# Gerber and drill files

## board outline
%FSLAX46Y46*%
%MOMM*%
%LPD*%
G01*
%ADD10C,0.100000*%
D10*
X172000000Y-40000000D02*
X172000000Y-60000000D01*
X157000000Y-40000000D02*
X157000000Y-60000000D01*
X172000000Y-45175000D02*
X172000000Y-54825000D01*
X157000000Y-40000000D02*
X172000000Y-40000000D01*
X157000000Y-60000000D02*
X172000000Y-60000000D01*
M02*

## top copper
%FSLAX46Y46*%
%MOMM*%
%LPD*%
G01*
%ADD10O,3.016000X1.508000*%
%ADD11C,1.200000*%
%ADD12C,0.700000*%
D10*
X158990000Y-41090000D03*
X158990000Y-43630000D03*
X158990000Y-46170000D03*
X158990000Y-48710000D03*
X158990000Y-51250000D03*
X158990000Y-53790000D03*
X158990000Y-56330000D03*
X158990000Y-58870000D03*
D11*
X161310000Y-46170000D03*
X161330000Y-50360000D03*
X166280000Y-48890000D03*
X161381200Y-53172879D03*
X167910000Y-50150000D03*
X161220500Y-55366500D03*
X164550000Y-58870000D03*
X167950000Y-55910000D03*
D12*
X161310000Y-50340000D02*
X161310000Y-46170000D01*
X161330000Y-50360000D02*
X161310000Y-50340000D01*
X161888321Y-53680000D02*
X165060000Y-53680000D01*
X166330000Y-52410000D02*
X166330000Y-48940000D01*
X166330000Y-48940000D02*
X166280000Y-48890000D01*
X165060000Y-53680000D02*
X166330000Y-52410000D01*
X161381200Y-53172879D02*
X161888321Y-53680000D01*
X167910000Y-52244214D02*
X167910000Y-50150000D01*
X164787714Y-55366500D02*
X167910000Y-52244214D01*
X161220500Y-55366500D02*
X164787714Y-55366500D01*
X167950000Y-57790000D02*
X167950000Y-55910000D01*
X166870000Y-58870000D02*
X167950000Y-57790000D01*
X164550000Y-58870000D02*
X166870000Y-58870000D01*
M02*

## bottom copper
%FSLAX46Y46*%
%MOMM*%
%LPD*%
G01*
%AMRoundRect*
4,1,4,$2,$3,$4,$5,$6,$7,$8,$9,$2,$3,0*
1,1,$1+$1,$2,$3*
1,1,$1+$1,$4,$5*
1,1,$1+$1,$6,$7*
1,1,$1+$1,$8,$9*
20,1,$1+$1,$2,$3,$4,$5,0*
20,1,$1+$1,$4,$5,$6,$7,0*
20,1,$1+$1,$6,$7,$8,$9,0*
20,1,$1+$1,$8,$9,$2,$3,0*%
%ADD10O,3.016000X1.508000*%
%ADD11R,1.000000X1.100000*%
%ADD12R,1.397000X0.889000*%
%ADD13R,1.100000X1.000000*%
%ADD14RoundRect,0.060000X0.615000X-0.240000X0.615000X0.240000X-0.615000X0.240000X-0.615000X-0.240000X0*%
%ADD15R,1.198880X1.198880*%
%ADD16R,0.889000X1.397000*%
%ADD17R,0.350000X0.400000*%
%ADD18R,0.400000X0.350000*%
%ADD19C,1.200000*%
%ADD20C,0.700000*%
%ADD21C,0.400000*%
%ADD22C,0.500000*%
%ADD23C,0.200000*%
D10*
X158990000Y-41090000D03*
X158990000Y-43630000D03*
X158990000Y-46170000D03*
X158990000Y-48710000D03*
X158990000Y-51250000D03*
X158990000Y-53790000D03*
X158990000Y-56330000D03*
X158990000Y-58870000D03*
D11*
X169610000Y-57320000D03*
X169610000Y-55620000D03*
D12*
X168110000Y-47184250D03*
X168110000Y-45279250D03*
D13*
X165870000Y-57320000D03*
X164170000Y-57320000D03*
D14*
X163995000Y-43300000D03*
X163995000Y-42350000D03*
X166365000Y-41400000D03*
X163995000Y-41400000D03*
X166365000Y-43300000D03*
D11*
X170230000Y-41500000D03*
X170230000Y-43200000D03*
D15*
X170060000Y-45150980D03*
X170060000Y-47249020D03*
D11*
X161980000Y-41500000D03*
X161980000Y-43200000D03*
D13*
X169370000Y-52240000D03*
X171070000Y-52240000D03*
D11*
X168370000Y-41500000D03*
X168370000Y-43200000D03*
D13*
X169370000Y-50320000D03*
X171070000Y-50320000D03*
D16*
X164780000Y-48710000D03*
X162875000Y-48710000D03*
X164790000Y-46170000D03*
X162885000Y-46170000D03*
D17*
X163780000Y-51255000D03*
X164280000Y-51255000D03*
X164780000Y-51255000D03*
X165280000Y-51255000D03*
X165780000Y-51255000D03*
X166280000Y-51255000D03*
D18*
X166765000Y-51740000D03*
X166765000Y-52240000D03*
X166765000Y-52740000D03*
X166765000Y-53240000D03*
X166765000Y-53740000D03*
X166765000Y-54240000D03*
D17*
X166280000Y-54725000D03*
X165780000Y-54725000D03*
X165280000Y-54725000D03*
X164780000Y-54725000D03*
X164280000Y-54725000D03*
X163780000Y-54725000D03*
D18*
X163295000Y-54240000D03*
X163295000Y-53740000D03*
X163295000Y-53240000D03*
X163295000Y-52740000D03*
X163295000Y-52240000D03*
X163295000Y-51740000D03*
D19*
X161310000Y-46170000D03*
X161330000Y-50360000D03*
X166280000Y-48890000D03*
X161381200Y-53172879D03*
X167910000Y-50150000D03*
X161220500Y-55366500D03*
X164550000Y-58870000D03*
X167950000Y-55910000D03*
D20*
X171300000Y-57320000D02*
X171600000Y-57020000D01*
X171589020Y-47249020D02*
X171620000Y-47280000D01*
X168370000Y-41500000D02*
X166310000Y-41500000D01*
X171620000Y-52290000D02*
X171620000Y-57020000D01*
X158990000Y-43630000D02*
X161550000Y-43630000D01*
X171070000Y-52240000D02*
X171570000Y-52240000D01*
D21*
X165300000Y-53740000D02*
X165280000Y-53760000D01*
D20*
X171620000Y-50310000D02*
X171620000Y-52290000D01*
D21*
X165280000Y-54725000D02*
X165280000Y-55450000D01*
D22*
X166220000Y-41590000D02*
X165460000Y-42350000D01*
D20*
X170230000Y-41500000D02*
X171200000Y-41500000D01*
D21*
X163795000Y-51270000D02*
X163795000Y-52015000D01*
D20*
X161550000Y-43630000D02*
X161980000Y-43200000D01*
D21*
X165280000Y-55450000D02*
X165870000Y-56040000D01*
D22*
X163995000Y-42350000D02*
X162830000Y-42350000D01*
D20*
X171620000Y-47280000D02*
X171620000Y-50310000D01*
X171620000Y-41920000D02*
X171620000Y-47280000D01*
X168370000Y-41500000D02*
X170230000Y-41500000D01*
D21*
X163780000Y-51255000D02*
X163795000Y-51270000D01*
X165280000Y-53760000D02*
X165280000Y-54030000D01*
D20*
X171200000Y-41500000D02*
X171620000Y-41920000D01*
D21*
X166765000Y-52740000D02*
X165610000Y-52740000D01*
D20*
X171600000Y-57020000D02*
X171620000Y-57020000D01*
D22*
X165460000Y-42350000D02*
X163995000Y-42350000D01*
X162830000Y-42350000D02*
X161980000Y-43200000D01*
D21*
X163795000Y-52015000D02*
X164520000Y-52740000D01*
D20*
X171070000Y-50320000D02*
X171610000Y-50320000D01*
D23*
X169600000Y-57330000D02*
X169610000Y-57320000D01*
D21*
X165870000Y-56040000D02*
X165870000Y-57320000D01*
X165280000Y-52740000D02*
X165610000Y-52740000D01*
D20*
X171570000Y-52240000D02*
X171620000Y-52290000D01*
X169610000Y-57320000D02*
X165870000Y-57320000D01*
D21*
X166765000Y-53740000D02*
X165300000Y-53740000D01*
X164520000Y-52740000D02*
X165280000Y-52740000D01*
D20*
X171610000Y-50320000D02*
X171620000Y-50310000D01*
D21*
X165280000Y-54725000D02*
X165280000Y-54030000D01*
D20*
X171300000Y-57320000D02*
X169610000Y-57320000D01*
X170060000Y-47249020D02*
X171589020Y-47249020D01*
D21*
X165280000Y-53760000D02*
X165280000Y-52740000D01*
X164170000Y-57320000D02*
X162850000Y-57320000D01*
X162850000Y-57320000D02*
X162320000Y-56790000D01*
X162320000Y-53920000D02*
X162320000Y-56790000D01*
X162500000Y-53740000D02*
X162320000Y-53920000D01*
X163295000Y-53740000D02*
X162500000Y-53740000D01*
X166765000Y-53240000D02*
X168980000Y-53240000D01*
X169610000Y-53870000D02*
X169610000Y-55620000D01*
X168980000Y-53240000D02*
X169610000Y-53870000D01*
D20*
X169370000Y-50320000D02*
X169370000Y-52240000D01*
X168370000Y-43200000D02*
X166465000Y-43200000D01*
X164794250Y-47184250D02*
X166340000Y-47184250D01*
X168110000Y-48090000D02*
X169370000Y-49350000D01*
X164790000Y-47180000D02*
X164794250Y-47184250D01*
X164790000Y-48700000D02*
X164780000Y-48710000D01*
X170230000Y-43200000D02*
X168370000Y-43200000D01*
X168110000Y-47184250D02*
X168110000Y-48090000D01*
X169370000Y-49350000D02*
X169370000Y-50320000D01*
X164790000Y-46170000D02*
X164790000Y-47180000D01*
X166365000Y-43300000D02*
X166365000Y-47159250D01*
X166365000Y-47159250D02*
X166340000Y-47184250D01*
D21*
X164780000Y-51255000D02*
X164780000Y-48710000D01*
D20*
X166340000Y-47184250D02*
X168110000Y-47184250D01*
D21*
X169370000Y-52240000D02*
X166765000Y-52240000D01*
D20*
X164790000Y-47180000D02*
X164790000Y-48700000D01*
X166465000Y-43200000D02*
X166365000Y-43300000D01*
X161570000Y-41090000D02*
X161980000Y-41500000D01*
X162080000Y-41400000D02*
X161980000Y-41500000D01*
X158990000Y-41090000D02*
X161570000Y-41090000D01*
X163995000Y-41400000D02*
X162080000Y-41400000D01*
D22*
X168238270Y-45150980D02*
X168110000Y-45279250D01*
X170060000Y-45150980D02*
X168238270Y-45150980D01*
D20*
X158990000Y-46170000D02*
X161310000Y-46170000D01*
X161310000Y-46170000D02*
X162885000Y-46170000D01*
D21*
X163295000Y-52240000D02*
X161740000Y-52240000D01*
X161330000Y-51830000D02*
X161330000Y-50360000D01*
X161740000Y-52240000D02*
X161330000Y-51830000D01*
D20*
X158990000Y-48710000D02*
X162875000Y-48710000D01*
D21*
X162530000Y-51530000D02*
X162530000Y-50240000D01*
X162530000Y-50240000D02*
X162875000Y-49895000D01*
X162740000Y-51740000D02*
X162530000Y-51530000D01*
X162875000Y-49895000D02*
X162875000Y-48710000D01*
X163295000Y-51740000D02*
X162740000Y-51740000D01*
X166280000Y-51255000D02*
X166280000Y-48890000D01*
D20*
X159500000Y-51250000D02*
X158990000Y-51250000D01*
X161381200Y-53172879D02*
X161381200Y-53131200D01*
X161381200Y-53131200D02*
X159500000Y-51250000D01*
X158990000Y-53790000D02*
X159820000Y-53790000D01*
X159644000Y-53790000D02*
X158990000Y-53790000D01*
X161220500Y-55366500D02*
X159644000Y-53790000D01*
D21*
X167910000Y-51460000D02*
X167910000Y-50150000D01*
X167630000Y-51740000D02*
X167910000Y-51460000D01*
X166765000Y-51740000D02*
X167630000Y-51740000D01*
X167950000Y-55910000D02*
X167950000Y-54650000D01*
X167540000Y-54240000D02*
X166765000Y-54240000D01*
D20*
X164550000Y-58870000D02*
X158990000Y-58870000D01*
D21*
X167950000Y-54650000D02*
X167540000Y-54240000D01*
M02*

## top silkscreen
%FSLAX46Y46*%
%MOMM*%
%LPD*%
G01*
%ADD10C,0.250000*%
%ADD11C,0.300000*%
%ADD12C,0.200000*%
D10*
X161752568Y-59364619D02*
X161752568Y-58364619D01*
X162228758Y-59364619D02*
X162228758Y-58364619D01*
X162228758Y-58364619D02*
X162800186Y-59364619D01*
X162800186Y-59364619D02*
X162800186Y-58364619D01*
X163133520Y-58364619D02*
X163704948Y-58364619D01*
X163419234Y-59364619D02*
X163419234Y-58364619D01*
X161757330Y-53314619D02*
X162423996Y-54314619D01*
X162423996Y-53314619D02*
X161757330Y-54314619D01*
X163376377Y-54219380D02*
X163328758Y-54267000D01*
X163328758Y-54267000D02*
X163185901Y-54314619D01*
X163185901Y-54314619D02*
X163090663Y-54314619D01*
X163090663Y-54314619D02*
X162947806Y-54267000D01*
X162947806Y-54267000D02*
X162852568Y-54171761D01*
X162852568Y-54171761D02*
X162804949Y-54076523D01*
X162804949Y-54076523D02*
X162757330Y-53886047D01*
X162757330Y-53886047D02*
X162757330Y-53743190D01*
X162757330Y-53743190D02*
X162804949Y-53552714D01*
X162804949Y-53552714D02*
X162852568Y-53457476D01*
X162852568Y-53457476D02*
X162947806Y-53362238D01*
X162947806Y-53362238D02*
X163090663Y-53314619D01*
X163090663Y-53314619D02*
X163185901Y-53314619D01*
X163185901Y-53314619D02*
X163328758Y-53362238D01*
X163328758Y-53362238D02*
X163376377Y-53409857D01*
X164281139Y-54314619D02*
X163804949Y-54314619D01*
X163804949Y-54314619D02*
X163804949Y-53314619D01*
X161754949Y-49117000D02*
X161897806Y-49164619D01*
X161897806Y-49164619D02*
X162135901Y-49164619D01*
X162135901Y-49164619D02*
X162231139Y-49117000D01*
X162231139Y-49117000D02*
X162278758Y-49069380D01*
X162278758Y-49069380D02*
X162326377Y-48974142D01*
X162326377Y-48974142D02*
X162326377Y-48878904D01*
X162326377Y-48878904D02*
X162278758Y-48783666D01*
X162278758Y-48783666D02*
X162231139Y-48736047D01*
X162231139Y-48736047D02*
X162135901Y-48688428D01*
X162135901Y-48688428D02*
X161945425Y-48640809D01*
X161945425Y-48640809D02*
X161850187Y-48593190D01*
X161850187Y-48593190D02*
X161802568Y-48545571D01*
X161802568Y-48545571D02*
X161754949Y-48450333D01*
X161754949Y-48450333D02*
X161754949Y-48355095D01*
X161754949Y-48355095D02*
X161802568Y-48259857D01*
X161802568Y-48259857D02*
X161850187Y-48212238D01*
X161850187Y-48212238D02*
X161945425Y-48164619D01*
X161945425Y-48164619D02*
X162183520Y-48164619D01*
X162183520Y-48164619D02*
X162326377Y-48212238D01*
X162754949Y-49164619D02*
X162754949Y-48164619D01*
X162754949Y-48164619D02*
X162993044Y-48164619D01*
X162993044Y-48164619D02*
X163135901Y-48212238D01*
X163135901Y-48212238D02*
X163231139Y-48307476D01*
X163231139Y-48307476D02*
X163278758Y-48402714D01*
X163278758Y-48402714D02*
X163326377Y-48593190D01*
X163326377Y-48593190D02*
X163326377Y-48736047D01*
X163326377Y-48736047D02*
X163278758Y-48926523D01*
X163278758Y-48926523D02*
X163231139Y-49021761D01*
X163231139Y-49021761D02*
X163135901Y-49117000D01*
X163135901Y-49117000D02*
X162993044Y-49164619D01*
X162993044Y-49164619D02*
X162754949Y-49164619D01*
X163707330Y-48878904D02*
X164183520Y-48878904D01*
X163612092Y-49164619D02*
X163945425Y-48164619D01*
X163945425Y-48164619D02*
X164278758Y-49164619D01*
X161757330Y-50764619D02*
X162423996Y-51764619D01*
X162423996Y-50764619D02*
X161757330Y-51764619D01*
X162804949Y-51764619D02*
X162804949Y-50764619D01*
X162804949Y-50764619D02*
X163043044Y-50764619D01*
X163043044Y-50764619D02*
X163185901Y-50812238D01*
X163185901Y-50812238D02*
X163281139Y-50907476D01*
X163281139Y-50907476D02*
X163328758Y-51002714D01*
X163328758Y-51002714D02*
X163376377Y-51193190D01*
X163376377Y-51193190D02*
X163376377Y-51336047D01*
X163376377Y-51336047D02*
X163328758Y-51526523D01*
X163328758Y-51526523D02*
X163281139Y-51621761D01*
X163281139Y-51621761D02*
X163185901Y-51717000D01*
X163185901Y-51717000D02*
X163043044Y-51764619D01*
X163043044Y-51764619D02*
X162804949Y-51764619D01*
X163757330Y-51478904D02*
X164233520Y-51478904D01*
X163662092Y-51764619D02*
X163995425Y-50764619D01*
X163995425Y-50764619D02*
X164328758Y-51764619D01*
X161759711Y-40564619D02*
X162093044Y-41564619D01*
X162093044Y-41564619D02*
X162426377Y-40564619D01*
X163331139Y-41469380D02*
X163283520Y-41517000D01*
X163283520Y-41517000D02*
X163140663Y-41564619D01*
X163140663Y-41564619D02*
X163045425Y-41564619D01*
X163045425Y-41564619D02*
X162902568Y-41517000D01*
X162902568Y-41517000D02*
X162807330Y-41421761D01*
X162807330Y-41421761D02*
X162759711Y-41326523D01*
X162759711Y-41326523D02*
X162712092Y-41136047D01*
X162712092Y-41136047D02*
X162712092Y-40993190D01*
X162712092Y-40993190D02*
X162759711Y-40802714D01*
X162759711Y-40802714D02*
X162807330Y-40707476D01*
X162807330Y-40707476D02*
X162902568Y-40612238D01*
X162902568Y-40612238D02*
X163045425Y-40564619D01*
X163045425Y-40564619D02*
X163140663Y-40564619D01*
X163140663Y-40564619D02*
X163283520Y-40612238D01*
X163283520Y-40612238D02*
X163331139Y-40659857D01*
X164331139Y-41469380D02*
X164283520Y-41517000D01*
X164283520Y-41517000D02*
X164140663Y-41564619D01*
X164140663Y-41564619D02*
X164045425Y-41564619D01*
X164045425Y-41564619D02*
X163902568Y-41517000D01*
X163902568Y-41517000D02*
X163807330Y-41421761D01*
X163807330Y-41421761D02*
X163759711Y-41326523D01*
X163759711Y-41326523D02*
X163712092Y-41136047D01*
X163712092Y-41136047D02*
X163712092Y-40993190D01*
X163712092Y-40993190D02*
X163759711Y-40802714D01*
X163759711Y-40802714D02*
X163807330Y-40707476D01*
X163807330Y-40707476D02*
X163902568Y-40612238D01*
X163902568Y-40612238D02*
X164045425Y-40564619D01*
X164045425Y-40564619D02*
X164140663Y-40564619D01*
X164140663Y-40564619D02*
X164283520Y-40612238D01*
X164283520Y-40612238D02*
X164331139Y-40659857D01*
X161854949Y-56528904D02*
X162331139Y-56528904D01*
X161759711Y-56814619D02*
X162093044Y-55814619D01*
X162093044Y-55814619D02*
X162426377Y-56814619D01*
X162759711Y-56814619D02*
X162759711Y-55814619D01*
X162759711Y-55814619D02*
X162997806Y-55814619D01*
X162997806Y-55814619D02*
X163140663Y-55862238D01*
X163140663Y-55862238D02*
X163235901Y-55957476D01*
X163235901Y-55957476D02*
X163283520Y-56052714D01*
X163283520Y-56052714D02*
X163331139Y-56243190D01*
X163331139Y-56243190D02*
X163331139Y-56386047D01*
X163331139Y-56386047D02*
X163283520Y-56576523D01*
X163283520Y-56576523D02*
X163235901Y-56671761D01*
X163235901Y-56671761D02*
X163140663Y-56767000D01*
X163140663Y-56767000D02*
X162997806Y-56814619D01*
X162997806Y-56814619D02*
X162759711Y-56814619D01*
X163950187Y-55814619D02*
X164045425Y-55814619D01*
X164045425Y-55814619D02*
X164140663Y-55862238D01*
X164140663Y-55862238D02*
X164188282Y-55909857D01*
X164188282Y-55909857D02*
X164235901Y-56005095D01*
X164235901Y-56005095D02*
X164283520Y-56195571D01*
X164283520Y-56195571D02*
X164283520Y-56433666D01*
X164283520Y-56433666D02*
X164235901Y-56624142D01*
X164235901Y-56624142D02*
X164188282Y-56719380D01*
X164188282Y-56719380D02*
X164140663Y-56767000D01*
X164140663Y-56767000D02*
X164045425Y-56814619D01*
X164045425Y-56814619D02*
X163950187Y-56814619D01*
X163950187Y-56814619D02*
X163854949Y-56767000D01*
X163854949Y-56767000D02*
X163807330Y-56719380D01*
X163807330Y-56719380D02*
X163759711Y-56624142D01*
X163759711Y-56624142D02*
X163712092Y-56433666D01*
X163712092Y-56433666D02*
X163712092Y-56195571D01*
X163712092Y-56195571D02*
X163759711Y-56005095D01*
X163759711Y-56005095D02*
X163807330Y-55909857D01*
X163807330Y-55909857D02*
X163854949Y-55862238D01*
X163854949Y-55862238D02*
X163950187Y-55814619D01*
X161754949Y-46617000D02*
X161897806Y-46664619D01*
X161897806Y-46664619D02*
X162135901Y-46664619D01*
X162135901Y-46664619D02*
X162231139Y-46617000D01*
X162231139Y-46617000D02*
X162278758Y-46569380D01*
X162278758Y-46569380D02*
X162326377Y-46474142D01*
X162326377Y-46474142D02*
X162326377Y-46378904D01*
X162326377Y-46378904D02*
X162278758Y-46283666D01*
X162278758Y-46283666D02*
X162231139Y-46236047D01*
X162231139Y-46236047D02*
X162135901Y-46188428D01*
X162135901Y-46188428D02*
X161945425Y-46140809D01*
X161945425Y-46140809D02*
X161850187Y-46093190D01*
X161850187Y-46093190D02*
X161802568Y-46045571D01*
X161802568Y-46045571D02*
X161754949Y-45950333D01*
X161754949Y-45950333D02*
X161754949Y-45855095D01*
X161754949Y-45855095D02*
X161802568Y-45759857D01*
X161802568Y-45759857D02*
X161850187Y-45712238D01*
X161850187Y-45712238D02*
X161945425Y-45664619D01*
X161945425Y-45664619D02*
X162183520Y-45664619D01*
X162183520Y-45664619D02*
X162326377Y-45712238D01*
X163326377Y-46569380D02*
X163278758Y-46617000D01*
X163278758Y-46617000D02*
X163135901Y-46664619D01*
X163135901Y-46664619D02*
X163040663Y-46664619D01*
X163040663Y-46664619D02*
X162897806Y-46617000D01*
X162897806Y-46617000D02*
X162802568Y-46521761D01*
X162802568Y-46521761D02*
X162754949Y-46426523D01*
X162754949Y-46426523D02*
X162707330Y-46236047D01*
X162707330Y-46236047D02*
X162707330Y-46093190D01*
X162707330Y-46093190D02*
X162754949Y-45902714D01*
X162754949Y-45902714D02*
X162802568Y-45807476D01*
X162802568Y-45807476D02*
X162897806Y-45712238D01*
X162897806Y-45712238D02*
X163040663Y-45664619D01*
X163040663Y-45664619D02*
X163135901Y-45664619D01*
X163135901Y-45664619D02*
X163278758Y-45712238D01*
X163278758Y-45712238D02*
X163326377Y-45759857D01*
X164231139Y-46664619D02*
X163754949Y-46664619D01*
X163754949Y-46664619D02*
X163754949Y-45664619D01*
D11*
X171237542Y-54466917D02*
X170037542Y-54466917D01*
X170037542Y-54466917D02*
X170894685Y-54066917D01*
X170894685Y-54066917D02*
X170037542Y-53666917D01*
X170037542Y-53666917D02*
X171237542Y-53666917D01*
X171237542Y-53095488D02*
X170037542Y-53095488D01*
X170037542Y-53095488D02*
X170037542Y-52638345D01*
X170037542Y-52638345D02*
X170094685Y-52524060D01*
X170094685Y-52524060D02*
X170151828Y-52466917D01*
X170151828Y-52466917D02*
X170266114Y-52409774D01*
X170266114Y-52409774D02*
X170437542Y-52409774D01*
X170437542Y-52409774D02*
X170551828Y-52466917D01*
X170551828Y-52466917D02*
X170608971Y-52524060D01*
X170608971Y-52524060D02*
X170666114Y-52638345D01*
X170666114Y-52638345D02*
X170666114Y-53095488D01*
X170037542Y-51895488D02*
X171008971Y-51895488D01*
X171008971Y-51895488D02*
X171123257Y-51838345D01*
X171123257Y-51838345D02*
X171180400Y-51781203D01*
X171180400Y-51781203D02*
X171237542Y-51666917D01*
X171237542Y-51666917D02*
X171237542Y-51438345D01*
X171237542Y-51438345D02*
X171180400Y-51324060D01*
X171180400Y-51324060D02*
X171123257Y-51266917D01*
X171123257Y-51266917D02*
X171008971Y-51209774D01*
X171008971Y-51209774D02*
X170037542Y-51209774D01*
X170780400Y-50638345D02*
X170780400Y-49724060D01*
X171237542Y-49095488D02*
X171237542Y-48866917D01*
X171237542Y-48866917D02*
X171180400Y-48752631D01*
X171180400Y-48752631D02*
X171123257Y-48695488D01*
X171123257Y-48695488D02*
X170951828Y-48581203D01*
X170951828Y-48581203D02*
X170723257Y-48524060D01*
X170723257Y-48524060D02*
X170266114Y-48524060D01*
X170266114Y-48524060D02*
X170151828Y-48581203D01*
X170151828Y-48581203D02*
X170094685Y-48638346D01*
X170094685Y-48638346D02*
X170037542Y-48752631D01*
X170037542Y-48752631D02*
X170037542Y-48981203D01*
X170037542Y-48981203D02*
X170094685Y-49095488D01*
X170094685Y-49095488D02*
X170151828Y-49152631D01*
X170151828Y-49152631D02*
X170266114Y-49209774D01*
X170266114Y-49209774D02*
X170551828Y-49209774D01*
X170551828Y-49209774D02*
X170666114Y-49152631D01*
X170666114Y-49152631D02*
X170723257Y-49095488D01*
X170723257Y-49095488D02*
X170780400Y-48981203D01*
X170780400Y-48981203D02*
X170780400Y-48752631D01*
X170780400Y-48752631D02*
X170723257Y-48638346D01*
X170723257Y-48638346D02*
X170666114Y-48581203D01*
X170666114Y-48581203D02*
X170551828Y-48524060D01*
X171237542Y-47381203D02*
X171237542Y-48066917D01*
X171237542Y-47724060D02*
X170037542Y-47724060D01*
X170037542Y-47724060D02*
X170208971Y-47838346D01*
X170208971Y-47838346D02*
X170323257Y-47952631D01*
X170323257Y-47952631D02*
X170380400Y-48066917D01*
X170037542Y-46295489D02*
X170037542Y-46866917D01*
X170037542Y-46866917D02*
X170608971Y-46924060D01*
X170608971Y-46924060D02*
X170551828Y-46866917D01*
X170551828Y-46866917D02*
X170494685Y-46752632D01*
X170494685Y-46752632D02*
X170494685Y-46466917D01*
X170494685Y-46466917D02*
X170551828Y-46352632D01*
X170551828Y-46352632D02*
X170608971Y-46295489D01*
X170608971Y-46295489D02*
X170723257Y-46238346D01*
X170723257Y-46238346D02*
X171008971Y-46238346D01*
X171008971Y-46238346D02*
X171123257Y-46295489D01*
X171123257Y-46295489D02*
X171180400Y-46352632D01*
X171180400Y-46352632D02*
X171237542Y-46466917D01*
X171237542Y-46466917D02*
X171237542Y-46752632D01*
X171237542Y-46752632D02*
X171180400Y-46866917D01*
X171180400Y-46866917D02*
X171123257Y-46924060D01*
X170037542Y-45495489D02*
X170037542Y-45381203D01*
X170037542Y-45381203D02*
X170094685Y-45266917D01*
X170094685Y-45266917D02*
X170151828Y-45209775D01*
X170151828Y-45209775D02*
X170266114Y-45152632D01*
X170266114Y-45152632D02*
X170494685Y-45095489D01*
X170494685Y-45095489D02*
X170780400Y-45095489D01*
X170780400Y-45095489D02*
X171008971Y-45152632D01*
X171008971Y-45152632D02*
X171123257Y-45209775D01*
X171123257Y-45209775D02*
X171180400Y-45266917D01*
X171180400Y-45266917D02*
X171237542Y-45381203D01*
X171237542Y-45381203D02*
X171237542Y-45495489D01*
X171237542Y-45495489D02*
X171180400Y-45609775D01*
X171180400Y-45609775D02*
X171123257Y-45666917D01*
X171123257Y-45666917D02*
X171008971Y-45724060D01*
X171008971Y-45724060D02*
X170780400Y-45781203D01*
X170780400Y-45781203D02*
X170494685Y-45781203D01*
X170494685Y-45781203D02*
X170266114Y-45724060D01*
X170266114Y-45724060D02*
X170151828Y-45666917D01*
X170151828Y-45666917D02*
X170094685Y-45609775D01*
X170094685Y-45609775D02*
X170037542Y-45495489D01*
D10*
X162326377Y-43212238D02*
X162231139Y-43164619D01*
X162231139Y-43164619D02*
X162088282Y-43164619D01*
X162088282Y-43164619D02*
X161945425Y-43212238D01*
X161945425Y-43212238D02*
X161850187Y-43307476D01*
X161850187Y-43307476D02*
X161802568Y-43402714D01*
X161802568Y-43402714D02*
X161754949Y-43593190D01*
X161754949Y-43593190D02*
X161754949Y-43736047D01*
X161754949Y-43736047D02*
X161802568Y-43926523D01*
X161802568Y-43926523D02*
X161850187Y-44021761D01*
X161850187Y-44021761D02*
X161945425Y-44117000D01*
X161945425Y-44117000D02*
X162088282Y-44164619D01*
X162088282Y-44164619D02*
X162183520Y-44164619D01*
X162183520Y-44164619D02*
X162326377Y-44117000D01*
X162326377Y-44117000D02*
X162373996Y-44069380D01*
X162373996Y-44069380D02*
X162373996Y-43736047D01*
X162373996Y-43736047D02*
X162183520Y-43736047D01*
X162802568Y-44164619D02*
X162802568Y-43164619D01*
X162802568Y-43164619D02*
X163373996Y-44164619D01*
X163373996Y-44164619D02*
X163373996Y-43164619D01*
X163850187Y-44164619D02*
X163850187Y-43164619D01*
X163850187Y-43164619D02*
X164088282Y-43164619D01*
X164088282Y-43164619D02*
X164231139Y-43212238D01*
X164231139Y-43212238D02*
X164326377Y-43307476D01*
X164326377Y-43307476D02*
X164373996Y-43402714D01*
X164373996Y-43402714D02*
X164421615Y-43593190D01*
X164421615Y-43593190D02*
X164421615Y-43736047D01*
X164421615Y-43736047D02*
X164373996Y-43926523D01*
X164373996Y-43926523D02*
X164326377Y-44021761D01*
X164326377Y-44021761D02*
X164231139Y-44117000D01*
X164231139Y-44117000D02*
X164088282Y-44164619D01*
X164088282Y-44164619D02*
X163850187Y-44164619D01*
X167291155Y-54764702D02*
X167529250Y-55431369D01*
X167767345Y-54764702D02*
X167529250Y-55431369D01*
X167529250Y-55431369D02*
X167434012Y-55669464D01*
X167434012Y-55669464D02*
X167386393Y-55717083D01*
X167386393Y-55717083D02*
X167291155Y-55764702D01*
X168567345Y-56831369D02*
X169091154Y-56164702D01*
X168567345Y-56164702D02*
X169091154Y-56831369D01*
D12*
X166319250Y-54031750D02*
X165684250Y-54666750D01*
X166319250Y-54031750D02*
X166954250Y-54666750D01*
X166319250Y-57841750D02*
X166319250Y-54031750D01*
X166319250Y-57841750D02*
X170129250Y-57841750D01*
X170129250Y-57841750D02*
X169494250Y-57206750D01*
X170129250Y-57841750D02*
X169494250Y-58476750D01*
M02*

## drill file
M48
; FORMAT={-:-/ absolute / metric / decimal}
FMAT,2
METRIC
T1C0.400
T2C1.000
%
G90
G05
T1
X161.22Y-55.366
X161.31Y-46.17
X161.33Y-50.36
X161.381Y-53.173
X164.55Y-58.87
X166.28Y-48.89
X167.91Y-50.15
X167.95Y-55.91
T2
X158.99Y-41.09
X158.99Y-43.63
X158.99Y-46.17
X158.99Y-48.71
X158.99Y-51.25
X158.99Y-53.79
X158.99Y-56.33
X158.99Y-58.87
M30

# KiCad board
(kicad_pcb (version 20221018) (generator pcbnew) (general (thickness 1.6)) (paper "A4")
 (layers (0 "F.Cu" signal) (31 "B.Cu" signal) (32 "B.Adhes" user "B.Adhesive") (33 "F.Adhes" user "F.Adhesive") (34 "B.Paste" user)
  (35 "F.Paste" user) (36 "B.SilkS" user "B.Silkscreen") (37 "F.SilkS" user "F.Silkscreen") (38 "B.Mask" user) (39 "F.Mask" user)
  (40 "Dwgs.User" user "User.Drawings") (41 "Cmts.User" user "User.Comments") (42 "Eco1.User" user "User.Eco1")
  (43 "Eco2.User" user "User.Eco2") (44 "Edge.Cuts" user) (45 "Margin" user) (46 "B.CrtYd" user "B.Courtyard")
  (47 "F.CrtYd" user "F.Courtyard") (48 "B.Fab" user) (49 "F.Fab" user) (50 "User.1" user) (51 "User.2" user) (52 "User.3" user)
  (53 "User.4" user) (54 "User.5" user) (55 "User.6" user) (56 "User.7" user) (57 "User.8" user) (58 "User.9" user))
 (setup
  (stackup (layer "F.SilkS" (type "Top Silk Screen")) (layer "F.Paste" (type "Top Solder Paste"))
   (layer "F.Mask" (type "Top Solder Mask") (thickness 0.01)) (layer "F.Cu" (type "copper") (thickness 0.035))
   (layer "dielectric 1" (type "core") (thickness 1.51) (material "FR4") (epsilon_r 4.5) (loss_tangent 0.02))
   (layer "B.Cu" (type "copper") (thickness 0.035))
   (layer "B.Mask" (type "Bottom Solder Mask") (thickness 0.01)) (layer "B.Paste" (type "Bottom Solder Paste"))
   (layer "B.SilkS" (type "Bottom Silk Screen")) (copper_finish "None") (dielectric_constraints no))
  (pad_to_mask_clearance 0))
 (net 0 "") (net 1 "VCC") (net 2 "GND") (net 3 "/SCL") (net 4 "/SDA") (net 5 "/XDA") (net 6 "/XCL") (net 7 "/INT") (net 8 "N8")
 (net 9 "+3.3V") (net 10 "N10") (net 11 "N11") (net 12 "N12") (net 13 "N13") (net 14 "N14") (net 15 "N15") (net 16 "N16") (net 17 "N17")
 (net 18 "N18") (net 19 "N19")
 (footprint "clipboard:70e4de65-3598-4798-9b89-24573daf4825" (layer "F.Cu") (at 170.12925 58.38175)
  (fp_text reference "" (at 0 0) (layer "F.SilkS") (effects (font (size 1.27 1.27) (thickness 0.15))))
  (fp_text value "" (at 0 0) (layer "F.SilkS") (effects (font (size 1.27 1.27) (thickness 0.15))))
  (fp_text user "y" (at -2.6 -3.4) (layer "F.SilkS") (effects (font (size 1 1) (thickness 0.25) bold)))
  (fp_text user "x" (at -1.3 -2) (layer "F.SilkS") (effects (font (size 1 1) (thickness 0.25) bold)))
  (fp_line (start -3.81 -4.35) (end -4.445 -3.715) (stroke (width 0.2) (type solid)) (layer "F.SilkS"))
  (fp_line (start -3.81 -4.35) (end -3.175 -3.715) (stroke (width 0.2) (type solid)) (layer "F.SilkS"))
  (fp_line (start -3.81 -0.54) (end -3.81 -4.35) (stroke (width 0.2) (type solid)) (layer "F.SilkS"))
  (fp_line (start -3.81 -0.54) (end 0 -0.54) (stroke (width 0.2) (type solid)) (layer "F.SilkS"))
  (fp_line (start 0 -0.54) (end -0.635 -1.175) (stroke (width 0.2) (type solid)) (layer "F.SilkS"))
  (fp_line (start 0 -0.54) (end -0.635 0.095) (stroke (width 0.2) (type solid)) (layer "F.SilkS")))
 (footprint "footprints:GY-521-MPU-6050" (layer "F.Cu") (at 158.99 50)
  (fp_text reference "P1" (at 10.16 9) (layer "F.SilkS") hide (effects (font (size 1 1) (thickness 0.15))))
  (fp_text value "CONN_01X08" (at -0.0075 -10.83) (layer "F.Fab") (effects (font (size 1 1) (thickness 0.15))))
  (pad "1" thru_hole oval (at 0 -8.91) (size 3.016 1.508) (drill 1) (layers "*.Cu" "*.Mask") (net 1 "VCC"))
  (pad "2" thru_hole oval (at 0 -6.37) (size 3.016 1.508) (drill 1) (layers "*.Cu" "*.Mask") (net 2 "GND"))
  (pad "3" thru_hole oval (at 0 -3.83) (size 3.016 1.508) (drill 1) (layers "*.Cu" "*.Mask") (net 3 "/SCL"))
  (pad "4" thru_hole oval (at 0 -1.29) (size 3.016 1.508) (drill 1) (layers "*.Cu" "*.Mask") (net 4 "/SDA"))
  (pad "5" thru_hole oval (at 0 1.25) (size 3.016 1.508) (drill 1) (layers "*.Cu" "*.Mask") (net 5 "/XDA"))
  (pad "6" thru_hole oval (at 0 3.79) (size 3.016 1.508) (drill 1) (layers "*.Cu" "*.Mask") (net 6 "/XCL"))
  (pad "7" thru_hole oval (at 0 6.33) (size 3.016 1.508) (drill 1) (layers "*.Cu" "*.Mask"))
  (pad "8" thru_hole oval (at 0 8.87) (size 3.016 1.508) (drill 1) (layers "*.Cu" "*.Mask") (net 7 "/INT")))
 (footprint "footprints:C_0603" (layer "B.Cu") (at 169.61 56.47 90)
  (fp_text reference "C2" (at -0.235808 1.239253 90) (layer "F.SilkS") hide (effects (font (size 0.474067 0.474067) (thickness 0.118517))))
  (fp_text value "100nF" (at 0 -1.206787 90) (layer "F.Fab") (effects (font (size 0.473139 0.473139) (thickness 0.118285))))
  (pad "1" smd rect (at -0.85 0 90) (size 1.1 1) (layers "B.Cu" "B.Paste" "B.Mask") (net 2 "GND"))
  (pad "2" smd rect (at 0.85 0 90) (size 1.1 1) (layers "B.Cu" "B.Paste" "B.Mask") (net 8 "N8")))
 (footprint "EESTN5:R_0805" (layer "B.Cu") (at 168.11 46.23175 90)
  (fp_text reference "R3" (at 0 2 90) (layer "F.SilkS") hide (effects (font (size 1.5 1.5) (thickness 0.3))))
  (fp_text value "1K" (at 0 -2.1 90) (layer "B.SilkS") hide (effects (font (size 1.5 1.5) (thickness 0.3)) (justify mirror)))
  (pad "1" smd rect (at -0.9525 0 90) (size 0.889 1.397) (layers "B.Cu" "B.Paste" "B.Mask") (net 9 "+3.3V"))
  (pad "2" smd rect (at 0.9525 0 90) (size 0.889 1.397) (layers "B.Cu" "B.Paste" "B.Mask") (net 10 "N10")))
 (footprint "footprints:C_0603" (layer "B.Cu") (at 165.02 57.32 180)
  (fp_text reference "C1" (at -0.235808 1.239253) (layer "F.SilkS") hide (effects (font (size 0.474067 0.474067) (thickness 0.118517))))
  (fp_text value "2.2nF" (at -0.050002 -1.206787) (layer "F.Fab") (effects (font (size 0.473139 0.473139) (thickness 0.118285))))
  (pad "1" smd rect (at -0.85 0 180) (size 1.1 1) (layers "B.Cu" "B.Paste" "B.Mask") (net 2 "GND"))
  (pad "2" smd rect (at 0.85 0 180) (size 1.1 1) (layers "B.Cu" "B.Paste" "B.Mask") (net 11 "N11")))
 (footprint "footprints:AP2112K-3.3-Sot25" (layer "B.Cu") (at 165.18 42.35)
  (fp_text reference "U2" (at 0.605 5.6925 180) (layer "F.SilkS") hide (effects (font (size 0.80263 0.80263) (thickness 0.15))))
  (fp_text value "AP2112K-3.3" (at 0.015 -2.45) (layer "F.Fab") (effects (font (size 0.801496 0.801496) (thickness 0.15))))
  (pad "1" smd roundrect (at -1.185 0.95 90) (size 0.6 1.35) (layers "B.Cu" "B.Paste" "B.Mask") (roundrect_rratio 0.1))
  (pad "2" smd roundrect (at -1.185 0 90) (size 0.6 1.35) (layers "B.Cu" "B.Paste" "B.Mask") (roundrect_rratio 0.1) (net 2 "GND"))
  (pad "2" smd roundrect (at 1.185 -0.95 90) (size 0.6 1.35) (layers "B.Cu" "B.Paste" "B.Mask") (roundrect_rratio 0.1) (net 2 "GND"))
  (pad "3" smd roundrect (at -1.185 -0.95 90) (size 0.6 1.35) (layers "B.Cu" "B.Paste" "B.Mask") (roundrect_rratio 0.1) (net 1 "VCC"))
  (pad "5" smd roundrect (at 1.185 0.95 90) (size 0.6 1.35) (layers "B.Cu" "B.Paste" "B.Mask") (roundrect_rratio 0.1) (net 9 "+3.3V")))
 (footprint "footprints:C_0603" (layer "B.Cu") (at 170.23 42.35 -90)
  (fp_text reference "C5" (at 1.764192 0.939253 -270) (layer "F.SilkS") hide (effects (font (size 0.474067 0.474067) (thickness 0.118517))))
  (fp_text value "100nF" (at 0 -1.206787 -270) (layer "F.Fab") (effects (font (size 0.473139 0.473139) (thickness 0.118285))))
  (pad "1" smd rect (at -0.85 0 270) (size 1.1 1) (layers "B.Cu" "B.Paste" "B.Mask") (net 2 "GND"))
  (pad "2" smd rect (at 0.85 0 270) (size 1.1 1) (layers "B.Cu" "B.Paste" "B.Mask") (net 9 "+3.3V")))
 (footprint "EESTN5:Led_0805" (layer "B.Cu") (at 170.06 46.2 -90)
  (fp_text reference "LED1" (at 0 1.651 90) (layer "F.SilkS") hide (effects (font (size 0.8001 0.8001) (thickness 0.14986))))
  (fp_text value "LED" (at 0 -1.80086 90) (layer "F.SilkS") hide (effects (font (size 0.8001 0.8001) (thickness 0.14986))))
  (pad "1" smd rect (at -1.04902 0 270) (size 1.19888 1.19888) (layers "B.Cu" "B.Paste" "B.Mask") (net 10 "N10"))
  (pad "2" smd rect (at 1.04902 0 270) (size 1.19888 1.19888) (layers "B.Cu" "B.Paste" "B.Mask") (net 2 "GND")))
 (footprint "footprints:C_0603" (layer "B.Cu") (at 161.98 42.35 -90)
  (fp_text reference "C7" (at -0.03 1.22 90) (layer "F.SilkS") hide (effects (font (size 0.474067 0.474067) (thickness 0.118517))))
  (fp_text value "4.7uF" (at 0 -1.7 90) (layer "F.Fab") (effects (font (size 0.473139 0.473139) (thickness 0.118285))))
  (pad "1" smd rect (at -0.85 0 270) (size 1.1 1) (layers "B.Cu" "B.Paste" "B.Mask") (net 1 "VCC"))
  (pad "2" smd rect (at 0.85 0 270) (size 1.1 1) (layers "B.Cu" "B.Paste" "B.Mask") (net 2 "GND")))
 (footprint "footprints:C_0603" (layer "B.Cu") (at 170.22 52.24)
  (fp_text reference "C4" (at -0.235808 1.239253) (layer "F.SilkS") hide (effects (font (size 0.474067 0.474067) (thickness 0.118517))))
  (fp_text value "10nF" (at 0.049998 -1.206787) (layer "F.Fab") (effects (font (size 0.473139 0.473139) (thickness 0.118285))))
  (pad "1" smd rect (at -0.85 0) (size 1.1 1) (layers "B.Cu" "B.Paste" "B.Mask") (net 9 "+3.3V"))
  (pad "2" smd rect (at 0.85 0) (size 1.1 1) (layers "B.Cu" "B.Paste" "B.Mask") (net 2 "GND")))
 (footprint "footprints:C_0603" (layer "B.Cu") (at 168.37 42.35 -90)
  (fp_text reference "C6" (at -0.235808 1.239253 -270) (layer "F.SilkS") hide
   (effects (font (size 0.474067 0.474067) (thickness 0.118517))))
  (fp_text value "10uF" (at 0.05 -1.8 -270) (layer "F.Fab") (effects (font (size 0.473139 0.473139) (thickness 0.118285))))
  (pad "1" smd rect (at -0.85 0 270) (size 1.1 1) (layers "B.Cu" "B.Paste" "B.Mask") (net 2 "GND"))
  (pad "2" smd rect (at 0.85 0 270) (size 1.1 1) (layers "B.Cu" "B.Paste" "B.Mask") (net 9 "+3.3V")))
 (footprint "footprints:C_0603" (layer "B.Cu") (at 170.22 50.32)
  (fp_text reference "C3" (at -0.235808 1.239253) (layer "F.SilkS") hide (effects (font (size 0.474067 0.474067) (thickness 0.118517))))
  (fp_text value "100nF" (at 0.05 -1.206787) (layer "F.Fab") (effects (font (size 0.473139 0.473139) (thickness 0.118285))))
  (pad "1" smd rect (at -0.85 0) (size 1.1 1) (layers "B.Cu" "B.Paste" "B.Mask") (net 9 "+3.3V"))
  (pad "2" smd rect (at 0.85 0) (size 1.1 1) (layers "B.Cu" "B.Paste" "B.Mask") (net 2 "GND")))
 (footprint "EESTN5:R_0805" (layer "B.Cu") (at 163.8275 48.71 180)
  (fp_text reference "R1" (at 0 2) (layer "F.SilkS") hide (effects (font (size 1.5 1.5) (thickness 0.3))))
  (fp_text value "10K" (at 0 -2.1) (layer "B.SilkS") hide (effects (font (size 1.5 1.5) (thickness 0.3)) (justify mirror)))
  (pad "1" smd rect (at -0.9525 0 180) (size 0.889 1.397) (layers "B.Cu" "B.Paste" "B.Mask") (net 9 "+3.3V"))
  (pad "2" smd rect (at 0.9525 0 180) (size 0.889 1.397) (layers "B.Cu" "B.Paste" "B.Mask") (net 4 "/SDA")))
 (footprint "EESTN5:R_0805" (layer "B.Cu") (at 163.8375 46.17 180)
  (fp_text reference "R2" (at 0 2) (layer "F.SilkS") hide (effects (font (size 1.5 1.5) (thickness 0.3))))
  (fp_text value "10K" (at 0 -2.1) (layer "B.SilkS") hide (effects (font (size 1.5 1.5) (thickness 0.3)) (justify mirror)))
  (pad "1" smd rect (at -0.9525 0 180) (size 0.889 1.397) (layers "B.Cu" "B.Paste" "B.Mask") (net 9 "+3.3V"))
  (pad "2" smd rect (at 0.9525 0 180) (size 0.889 1.397) (layers "B.Cu" "B.Paste" "B.Mask") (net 3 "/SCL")))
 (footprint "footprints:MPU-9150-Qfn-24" (layer "B.Cu") (at 165.03 52.99 -90)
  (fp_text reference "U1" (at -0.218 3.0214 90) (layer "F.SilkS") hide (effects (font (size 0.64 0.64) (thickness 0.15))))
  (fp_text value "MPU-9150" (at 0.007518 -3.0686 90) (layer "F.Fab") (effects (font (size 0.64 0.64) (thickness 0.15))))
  (pad "1" smd rect (at -1.735 1.25 270) (size 0.4 0.35) (layers "B.Cu" "B.Paste") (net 2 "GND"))
  (pad "2" smd rect (at -1.735 0.75 270) (size 0.4 0.35) (layers "B.Cu" "B.Paste") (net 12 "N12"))
  (pad "3" smd rect (at -1.735 0.25 270) (size 0.4 0.35) (layers "B.Cu" "B.Paste") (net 9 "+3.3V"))
  (pad "4" smd rect (at -1.735 -0.25 270) (size 0.4 0.35) (layers "B.Cu" "B.Paste") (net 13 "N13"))
  (pad "5" smd rect (at -1.735 -0.75 270) (size 0.4 0.35) (layers "B.Cu" "B.Paste") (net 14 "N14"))
  (pad "6" smd rect (at -1.735 -1.25 270) (size 0.4 0.35) (layers "B.Cu" "B.Paste") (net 5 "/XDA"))
  (pad "7" smd rect (at -1.25 -1.735 270) (size 0.35 0.4) (layers "B.Cu" "B.Paste") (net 6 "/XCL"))
  (pad "8" smd rect (at -0.75 -1.735 270) (size 0.35 0.4) (layers "B.Cu" "B.Paste") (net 9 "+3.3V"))
  (pad "9" smd rect (at -0.25 -1.735 270) (size 0.35 0.4) (layers "B.Cu" "B.Paste") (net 2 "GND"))
  (pad "10" smd rect (at 0.25 -1.735 270) (size 0.35 0.4) (layers "B.Cu" "B.Paste") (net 8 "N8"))
  (pad "11" smd rect (at 0.75 -1.735 270) (size 0.35 0.4) (layers "B.Cu" "B.Paste") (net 2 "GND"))
  (pad "12" smd rect (at 1.25 -1.735 270) (size 0.35 0.4) (layers "B.Cu" "B.Paste") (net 7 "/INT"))
  (pad "13" smd rect (at 1.735 -1.25 270) (size 0.4 0.35) (layers "B.Cu" "B.Paste"))
  (pad "14" smd rect (at 1.735 -0.75 270) (size 0.4 0.35) (layers "B.Cu" "B.Paste") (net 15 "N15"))
  (pad "15" smd rect (at 1.735 -0.25 270) (size 0.4 0.35) (layers "B.Cu" "B.Paste") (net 2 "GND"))
  (pad "16" smd rect (at 1.735 0.25 270) (size 0.4 0.35) (layers "B.Cu" "B.Paste") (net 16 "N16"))
  (pad "17" smd rect (at 1.735 0.75 270) (size 0.4 0.35) (layers "B.Cu" "B.Paste"))
  (pad "18" smd rect (at 1.735 1.25 270) (size 0.4 0.35) (layers "B.Cu" "B.Paste"))
  (pad "19" smd rect (at 1.25 1.735 270) (size 0.35 0.4) (layers "B.Cu" "B.Paste") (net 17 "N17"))
  (pad "20" smd rect (at 0.75 1.735 270) (size 0.35 0.4) (layers "B.Cu" "B.Paste") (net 11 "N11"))
  (pad "21" smd rect (at 0.25 1.735 270) (size 0.35 0.4) (layers "B.Cu" "B.Paste") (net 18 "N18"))
  (pad "22" smd rect (at -0.25 1.735 270) (size 0.35 0.4) (layers "B.Cu" "B.Paste") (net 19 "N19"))
  (pad "23" smd rect (at -0.75 1.735 270) (size 0.35 0.4) (layers "B.Cu" "B.Paste") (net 3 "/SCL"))
  (pad "24" smd rect (at -1.25 1.735 270) (size 0.35 0.4) (layers "B.Cu" "B.Paste") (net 4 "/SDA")))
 (gr_line (start 172 40) (end 172 60) (stroke (width 0.1) (type default)) (layer "Edge.Cuts"))
 (gr_line (start 157 40) (end 157 60) (stroke (width 0.1) (type default)) (layer "Edge.Cuts"))
 (gr_line (start 172 45.175) (end 172 54.825) (stroke (width 0.1) (type default)) (layer "Edge.Cuts"))
 (gr_line (start 157 40) (end 172 40) (stroke (width 0.1) (type default)) (layer "Edge.Cuts"))
 (gr_line (start 157 60) (end 172 60) (stroke (width 0.1) (type default)) (layer "Edge.Cuts"))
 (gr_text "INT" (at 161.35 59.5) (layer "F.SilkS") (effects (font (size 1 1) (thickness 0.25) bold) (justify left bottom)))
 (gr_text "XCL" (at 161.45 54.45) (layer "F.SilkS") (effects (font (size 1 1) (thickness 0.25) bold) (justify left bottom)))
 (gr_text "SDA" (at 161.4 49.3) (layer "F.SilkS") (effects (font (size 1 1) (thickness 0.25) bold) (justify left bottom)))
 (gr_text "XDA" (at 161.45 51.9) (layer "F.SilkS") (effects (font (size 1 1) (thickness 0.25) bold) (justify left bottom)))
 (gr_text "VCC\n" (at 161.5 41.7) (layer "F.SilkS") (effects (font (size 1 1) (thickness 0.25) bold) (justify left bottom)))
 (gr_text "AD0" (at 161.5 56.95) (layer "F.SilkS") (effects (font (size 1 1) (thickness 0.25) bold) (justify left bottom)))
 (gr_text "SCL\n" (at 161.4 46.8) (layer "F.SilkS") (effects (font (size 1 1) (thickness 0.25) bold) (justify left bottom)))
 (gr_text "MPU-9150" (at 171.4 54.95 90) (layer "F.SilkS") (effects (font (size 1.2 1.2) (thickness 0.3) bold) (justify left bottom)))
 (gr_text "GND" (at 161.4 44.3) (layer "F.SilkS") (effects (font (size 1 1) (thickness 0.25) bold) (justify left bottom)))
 (segment (start 171.3 57.32) (end 171.6 57.02) (width 0.7) (layer "B.Cu") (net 2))
 (segment (start 171.58902 47.24902) (end 171.62 47.28) (width 0.7) (layer "B.Cu") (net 2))
 (segment (start 168.37 41.5) (end 166.31 41.5) (width 0.7) (layer "B.Cu") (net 2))
 (segment (start 171.62 52.29) (end 171.62 57.02) (width 0.7) (layer "B.Cu") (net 2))
 (segment (start 158.99 43.63) (end 161.55 43.63) (width 0.7) (layer "B.Cu") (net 2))
 (segment (start 171.07 52.24) (end 171.57 52.24) (width 0.7) (layer "B.Cu") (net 2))
 (segment (start 165.3 53.74) (end 165.28 53.76) (width 0.4) (layer "B.Cu") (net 2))
 (segment (start 171.62 50.31) (end 171.62 52.29) (width 0.7) (layer "B.Cu") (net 2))
 (segment (start 165.28 54.725) (end 165.28 55.45) (width 0.4) (layer "B.Cu") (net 2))
 (segment (start 166.22 41.59) (end 165.46 42.35) (width 0.5) (layer "B.Cu") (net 2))
 (segment (start 170.23 41.5) (end 171.2 41.5) (width 0.7) (layer "B.Cu") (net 2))
 (segment (start 163.795 51.27) (end 163.795 52.015) (width 0.4) (layer "B.Cu") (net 2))
 (segment (start 161.55 43.63) (end 161.98 43.2) (width 0.7) (layer "B.Cu") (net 2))
 (segment (start 165.28 55.45) (end 165.87 56.04) (width 0.4) (layer "B.Cu") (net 2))
 (segment (start 163.995 42.35) (end 162.83 42.35) (width 0.5) (layer "B.Cu") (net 2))
 (segment (start 171.62 47.28) (end 171.62 50.31) (width 0.7) (layer "B.Cu") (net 2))
 (segment (start 171.62 41.92) (end 171.62 47.28) (width 0.7) (layer "B.Cu") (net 2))
 (segment (start 168.37 41.5) (end 170.23 41.5) (width 0.7) (layer "B.Cu") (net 2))
 (segment (start 163.78 51.255) (end 163.795 51.27) (width 0.4) (layer "B.Cu") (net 2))
 (segment (start 165.28 53.76) (end 165.28 54.03) (width 0.4) (layer "B.Cu") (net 2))
 (segment (start 171.2 41.5) (end 171.62 41.92) (width 0.7) (layer "B.Cu") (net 2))
 (segment (start 166.765 52.74) (end 165.61 52.74) (width 0.4) (layer "B.Cu") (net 2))
 (segment (start 171.6 57.02) (end 171.62 57.02) (width 0.7) (layer "B.Cu") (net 2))
 (segment (start 165.46 42.35) (end 163.995 42.35) (width 0.5) (layer "B.Cu") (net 2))
 (segment (start 162.83 42.35) (end 161.98 43.2) (width 0.5) (layer "B.Cu") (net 2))
 (segment (start 163.795 52.015) (end 164.52 52.74) (width 0.4) (layer "B.Cu") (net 2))
 (segment (start 171.07 50.32) (end 171.61 50.32) (width 0.7) (layer "B.Cu") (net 2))
 (segment (start 169.6 57.33) (end 169.61 57.32) (width 0.2) (layer "B.Cu") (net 2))
 (segment (start 165.87 56.04) (end 165.87 57.32) (width 0.4) (layer "B.Cu") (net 2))
 (segment (start 165.28 52.74) (end 165.61 52.74) (width 0.4) (layer "B.Cu") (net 2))
 (segment (start 171.57 52.24) (end 171.62 52.29) (width 0.7) (layer "B.Cu") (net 2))
 (segment (start 169.61 57.32) (end 165.87 57.32) (width 0.7) (layer "B.Cu") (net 2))
 (segment (start 166.765 53.74) (end 165.3 53.74) (width 0.4) (layer "B.Cu") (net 2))
 (segment (start 164.52 52.74) (end 165.28 52.74) (width 0.4) (layer "B.Cu") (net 2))
 (segment (start 171.61 50.32) (end 171.62 50.31) (width 0.7) (layer "B.Cu") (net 2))
 (segment (start 165.28 54.725) (end 165.28 54.03) (width 0.4) (layer "B.Cu") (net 2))
 (segment (start 171.3 57.32) (end 169.61 57.32) (width 0.7) (layer "B.Cu") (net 2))
 (segment (start 170.06 47.24902) (end 171.58902 47.24902) (width 0.7) (layer "B.Cu") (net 2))
 (segment (start 165.28 53.76) (end 165.28 52.74) (width 0.4) (layer "B.Cu") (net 2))
 (segment (start 164.17 57.32) (end 162.85 57.32) (width 0.4) (layer "B.Cu") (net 11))
 (segment (start 162.85 57.32) (end 162.32 56.79) (width 0.4) (layer "B.Cu") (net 11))
 (segment (start 162.32 53.92) (end 162.32 56.79) (width 0.4) (layer "B.Cu") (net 11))
 (segment (start 162.5 53.74) (end 162.32 53.92) (width 0.4) (layer "B.Cu") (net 11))
 (segment (start 163.295 53.74) (end 162.5 53.74) (width 0.4) (layer "B.Cu") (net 11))
 (segment (start 166.765 53.24) (end 168.98 53.24) (width 0.4) (layer "B.Cu") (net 8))
 (segment (start 169.61 53.87) (end 169.61 55.62) (width 0.4) (layer "B.Cu") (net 8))
 (segment (start 168.98 53.24) (end 169.61 53.87) (width 0.4) (layer "B.Cu") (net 8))
 (segment (start 169.37 50.32) (end 169.37 52.24) (width 0.7) (layer "B.Cu") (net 9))
 (segment (start 168.37 43.2) (end 166.465 43.2) (width 0.7) (layer "B.Cu") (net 9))
 (segment (start 164.79425 47.18425) (end 166.34 47.18425) (width 0.7) (layer "B.Cu") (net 9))
 (segment (start 168.11 48.09) (end 169.37 49.35) (width 0.7) (layer "B.Cu") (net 9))
 (segment (start 164.79 47.18) (end 164.79425 47.18425) (width 0.7) (layer "B.Cu") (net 9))
 (segment (start 164.79 48.7) (end 164.78 48.71) (width 0.7) (layer "B.Cu") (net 9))
 (segment (start 170.23 43.2) (end 168.37 43.2) (width 0.7) (layer "B.Cu") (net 9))
 (segment (start 168.11 47.18425) (end 168.11 48.09) (width 0.7) (layer "B.Cu") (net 9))
 (segment (start 169.37 49.35) (end 169.37 50.32) (width 0.7) (layer "B.Cu") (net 9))
 (segment (start 164.79 46.17) (end 164.79 47.18) (width 0.7) (layer "B.Cu") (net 9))
 (segment (start 166.365 43.3) (end 166.365 47.15925) (width 0.7) (layer "B.Cu") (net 9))
 (segment (start 166.365 47.15925) (end 166.34 47.18425) (width 0.7) (layer "B.Cu") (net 9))
 (segment (start 164.78 51.255) (end 164.78 48.71) (width 0.4) (layer "B.Cu") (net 9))
 (segment (start 166.34 47.18425) (end 168.11 47.18425) (width 0.7) (layer "B.Cu") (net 9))
 (segment (start 169.37 52.24) (end 166.765 52.24) (width 0.4) (layer "B.Cu") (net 9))
 (segment (start 164.79 47.18) (end 164.79 48.7) (width 0.7) (layer "B.Cu") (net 9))
 (segment (start 166.465 43.2) (end 166.365 43.3) (width 0.7) (layer "B.Cu") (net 9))
 (segment (start 161.57 41.09) (end 161.98 41.5) (width 0.7) (layer "B.Cu") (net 1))
 (segment (start 162.08 41.4) (end 161.98 41.5) (width 0.7) (layer "B.Cu") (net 1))
 (segment (start 158.99 41.09) (end 161.57 41.09) (width 0.7) (layer "B.Cu") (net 1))
 (segment (start 163.995 41.4) (end 162.08 41.4) (width 0.7) (layer "B.Cu") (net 1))
 (segment (start 168.23827 45.15098) (end 168.11 45.27925) (width 0.5) (layer "B.Cu") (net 10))
 (segment (start 170.06 45.15098) (end 168.23827 45.15098) (width 0.5) (layer "B.Cu") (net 10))
 (segment (start 161.31 50.34) (end 161.31 46.17) (width 0.7) (layer "F.Cu") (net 3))
 (segment (start 161.33 50.36) (end 161.31 50.34) (width 0.7) (layer "F.Cu") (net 3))
 (via (at 161.31 46.17) (size 1.2) (drill 0.4) (layers "F.Cu" "B.Cu") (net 3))
 (via (at 161.33 50.36) (size 1.2) (drill 0.4) (layers "F.Cu" "B.Cu") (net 3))
 (segment (start 158.99 46.17) (end 161.31 46.17) (width 0.7) (layer "B.Cu") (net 3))
 (segment (start 161.31 46.17) (end 162.885 46.17) (width 0.7) (layer "B.Cu") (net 3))
 (segment (start 163.295 52.24) (end 161.74 52.24) (width 0.4) (layer "B.Cu") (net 3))
 (segment (start 161.33 51.83) (end 161.33 50.36) (width 0.4) (layer "B.Cu") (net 3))
 (segment (start 161.74 52.24) (end 161.33 51.83) (width 0.4) (layer "B.Cu") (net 3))
 (segment (start 158.99 48.71) (end 162.875 48.71) (width 0.7) (layer "B.Cu") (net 4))
 (segment (start 162.53 51.53) (end 162.53 50.24) (width 0.4) (layer "B.Cu") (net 4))
 (segment (start 162.53 50.24) (end 162.875 49.895) (width 0.4) (layer "B.Cu") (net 4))
 (segment (start 162.74 51.74) (end 162.53 51.53) (width 0.4) (layer "B.Cu") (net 4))
 (segment (start 162.875 49.895) (end 162.875 48.71) (width 0.4) (layer "B.Cu") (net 4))
 (segment (start 163.295 51.74) (end 162.74 51.74) (width 0.4) (layer "B.Cu") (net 4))
 (segment (start 161.888321 53.68) (end 165.06 53.68) (width 0.7) (layer "F.Cu") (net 5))
 (segment (start 166.33 52.41) (end 166.33 48.94) (width 0.7) (layer "F.Cu") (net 5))
 (segment (start 166.33 48.94) (end 166.28 48.89) (width 0.7) (layer "F.Cu") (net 5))
 (segment (start 165.06 53.68) (end 166.33 52.41) (width 0.7) (layer "F.Cu") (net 5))
 (segment (start 161.3812 53.172879) (end 161.888321 53.68) (width 0.7) (layer "F.Cu") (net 5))
 (via (at 166.28 48.89) (size 1.2) (drill 0.4) (layers "F.Cu" "B.Cu") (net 5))
 (via (at 161.3812 53.172879) (size 1.2) (drill 0.4) (layers "F.Cu" "B.Cu") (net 5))
 (segment (start 166.28 51.255) (end 166.28 48.89) (width 0.4) (layer "B.Cu") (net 5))
 (segment (start 159.5 51.25) (end 158.99 51.25) (width 0.7) (layer "B.Cu") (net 5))
 (segment (start 161.3812 53.172879) (end 161.3812 53.1312) (width 0.7) (layer "B.Cu") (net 5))
 (segment (start 161.3812 53.1312) (end 159.5 51.25) (width 0.7) (layer "B.Cu") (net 5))
 (segment (start 167.91 52.244214) (end 167.91 50.15) (width 0.7) (layer "F.Cu") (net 6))
 (segment (start 164.787714 55.3665) (end 167.91 52.244214) (width 0.7) (layer "F.Cu") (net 6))
 (segment (start 161.2205 55.3665) (end 164.787714 55.3665) (width 0.7) (layer "F.Cu") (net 6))
 (via (at 167.91 50.15) (size 1.2) (drill 0.4) (layers "F.Cu" "B.Cu") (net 6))
 (via (at 161.2205 55.3665) (size 1.2) (drill 0.4) (layers "F.Cu" "B.Cu") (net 6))
 (segment (start 158.99 53.79) (end 159.82 53.79) (width 0.7) (layer "B.Cu") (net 6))
 (segment (start 159.644 53.79) (end 158.99 53.79) (width 0.7) (layer "B.Cu") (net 6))
 (segment (start 161.2205 55.3665) (end 159.644 53.79) (width 0.7) (layer "B.Cu") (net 6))
 (segment (start 167.91 51.46) (end 167.91 50.15) (width 0.4) (layer "B.Cu") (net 6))
 (segment (start 167.63 51.74) (end 167.91 51.46) (width 0.4) (layer "B.Cu") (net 6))
 (segment (start 166.765 51.74) (end 167.63 51.74) (width 0.4) (layer "B.Cu") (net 6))
 (segment (start 167.95 57.79) (end 167.95 55.91) (width 0.7) (layer "F.Cu") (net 7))
 (segment (start 166.87 58.87) (end 167.95 57.79) (width 0.7) (layer "F.Cu") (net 7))
 (segment (start 164.55 58.87) (end 166.87 58.87) (width 0.7) (layer "F.Cu") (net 7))
 (via (at 164.55 58.87) (size 1.2) (drill 0.4) (layers "F.Cu" "B.Cu") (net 7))
 (via (at 167.95 55.91) (size 1.2) (drill 0.4) (layers "F.Cu" "B.Cu") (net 7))
 (segment (start 167.95 55.91) (end 167.95 54.65) (width 0.4) (layer "B.Cu") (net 7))
 (segment (start 167.54 54.24) (end 166.765 54.24) (width 0.4) (layer "B.Cu") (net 7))
 (segment (start 164.55 58.87) (end 158.99 58.87) (width 0.7) (layer "B.Cu") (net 7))
 (segment (start 167.95 54.65) (end 167.54 54.24) (width 0.4) (layer "B.Cu") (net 7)))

